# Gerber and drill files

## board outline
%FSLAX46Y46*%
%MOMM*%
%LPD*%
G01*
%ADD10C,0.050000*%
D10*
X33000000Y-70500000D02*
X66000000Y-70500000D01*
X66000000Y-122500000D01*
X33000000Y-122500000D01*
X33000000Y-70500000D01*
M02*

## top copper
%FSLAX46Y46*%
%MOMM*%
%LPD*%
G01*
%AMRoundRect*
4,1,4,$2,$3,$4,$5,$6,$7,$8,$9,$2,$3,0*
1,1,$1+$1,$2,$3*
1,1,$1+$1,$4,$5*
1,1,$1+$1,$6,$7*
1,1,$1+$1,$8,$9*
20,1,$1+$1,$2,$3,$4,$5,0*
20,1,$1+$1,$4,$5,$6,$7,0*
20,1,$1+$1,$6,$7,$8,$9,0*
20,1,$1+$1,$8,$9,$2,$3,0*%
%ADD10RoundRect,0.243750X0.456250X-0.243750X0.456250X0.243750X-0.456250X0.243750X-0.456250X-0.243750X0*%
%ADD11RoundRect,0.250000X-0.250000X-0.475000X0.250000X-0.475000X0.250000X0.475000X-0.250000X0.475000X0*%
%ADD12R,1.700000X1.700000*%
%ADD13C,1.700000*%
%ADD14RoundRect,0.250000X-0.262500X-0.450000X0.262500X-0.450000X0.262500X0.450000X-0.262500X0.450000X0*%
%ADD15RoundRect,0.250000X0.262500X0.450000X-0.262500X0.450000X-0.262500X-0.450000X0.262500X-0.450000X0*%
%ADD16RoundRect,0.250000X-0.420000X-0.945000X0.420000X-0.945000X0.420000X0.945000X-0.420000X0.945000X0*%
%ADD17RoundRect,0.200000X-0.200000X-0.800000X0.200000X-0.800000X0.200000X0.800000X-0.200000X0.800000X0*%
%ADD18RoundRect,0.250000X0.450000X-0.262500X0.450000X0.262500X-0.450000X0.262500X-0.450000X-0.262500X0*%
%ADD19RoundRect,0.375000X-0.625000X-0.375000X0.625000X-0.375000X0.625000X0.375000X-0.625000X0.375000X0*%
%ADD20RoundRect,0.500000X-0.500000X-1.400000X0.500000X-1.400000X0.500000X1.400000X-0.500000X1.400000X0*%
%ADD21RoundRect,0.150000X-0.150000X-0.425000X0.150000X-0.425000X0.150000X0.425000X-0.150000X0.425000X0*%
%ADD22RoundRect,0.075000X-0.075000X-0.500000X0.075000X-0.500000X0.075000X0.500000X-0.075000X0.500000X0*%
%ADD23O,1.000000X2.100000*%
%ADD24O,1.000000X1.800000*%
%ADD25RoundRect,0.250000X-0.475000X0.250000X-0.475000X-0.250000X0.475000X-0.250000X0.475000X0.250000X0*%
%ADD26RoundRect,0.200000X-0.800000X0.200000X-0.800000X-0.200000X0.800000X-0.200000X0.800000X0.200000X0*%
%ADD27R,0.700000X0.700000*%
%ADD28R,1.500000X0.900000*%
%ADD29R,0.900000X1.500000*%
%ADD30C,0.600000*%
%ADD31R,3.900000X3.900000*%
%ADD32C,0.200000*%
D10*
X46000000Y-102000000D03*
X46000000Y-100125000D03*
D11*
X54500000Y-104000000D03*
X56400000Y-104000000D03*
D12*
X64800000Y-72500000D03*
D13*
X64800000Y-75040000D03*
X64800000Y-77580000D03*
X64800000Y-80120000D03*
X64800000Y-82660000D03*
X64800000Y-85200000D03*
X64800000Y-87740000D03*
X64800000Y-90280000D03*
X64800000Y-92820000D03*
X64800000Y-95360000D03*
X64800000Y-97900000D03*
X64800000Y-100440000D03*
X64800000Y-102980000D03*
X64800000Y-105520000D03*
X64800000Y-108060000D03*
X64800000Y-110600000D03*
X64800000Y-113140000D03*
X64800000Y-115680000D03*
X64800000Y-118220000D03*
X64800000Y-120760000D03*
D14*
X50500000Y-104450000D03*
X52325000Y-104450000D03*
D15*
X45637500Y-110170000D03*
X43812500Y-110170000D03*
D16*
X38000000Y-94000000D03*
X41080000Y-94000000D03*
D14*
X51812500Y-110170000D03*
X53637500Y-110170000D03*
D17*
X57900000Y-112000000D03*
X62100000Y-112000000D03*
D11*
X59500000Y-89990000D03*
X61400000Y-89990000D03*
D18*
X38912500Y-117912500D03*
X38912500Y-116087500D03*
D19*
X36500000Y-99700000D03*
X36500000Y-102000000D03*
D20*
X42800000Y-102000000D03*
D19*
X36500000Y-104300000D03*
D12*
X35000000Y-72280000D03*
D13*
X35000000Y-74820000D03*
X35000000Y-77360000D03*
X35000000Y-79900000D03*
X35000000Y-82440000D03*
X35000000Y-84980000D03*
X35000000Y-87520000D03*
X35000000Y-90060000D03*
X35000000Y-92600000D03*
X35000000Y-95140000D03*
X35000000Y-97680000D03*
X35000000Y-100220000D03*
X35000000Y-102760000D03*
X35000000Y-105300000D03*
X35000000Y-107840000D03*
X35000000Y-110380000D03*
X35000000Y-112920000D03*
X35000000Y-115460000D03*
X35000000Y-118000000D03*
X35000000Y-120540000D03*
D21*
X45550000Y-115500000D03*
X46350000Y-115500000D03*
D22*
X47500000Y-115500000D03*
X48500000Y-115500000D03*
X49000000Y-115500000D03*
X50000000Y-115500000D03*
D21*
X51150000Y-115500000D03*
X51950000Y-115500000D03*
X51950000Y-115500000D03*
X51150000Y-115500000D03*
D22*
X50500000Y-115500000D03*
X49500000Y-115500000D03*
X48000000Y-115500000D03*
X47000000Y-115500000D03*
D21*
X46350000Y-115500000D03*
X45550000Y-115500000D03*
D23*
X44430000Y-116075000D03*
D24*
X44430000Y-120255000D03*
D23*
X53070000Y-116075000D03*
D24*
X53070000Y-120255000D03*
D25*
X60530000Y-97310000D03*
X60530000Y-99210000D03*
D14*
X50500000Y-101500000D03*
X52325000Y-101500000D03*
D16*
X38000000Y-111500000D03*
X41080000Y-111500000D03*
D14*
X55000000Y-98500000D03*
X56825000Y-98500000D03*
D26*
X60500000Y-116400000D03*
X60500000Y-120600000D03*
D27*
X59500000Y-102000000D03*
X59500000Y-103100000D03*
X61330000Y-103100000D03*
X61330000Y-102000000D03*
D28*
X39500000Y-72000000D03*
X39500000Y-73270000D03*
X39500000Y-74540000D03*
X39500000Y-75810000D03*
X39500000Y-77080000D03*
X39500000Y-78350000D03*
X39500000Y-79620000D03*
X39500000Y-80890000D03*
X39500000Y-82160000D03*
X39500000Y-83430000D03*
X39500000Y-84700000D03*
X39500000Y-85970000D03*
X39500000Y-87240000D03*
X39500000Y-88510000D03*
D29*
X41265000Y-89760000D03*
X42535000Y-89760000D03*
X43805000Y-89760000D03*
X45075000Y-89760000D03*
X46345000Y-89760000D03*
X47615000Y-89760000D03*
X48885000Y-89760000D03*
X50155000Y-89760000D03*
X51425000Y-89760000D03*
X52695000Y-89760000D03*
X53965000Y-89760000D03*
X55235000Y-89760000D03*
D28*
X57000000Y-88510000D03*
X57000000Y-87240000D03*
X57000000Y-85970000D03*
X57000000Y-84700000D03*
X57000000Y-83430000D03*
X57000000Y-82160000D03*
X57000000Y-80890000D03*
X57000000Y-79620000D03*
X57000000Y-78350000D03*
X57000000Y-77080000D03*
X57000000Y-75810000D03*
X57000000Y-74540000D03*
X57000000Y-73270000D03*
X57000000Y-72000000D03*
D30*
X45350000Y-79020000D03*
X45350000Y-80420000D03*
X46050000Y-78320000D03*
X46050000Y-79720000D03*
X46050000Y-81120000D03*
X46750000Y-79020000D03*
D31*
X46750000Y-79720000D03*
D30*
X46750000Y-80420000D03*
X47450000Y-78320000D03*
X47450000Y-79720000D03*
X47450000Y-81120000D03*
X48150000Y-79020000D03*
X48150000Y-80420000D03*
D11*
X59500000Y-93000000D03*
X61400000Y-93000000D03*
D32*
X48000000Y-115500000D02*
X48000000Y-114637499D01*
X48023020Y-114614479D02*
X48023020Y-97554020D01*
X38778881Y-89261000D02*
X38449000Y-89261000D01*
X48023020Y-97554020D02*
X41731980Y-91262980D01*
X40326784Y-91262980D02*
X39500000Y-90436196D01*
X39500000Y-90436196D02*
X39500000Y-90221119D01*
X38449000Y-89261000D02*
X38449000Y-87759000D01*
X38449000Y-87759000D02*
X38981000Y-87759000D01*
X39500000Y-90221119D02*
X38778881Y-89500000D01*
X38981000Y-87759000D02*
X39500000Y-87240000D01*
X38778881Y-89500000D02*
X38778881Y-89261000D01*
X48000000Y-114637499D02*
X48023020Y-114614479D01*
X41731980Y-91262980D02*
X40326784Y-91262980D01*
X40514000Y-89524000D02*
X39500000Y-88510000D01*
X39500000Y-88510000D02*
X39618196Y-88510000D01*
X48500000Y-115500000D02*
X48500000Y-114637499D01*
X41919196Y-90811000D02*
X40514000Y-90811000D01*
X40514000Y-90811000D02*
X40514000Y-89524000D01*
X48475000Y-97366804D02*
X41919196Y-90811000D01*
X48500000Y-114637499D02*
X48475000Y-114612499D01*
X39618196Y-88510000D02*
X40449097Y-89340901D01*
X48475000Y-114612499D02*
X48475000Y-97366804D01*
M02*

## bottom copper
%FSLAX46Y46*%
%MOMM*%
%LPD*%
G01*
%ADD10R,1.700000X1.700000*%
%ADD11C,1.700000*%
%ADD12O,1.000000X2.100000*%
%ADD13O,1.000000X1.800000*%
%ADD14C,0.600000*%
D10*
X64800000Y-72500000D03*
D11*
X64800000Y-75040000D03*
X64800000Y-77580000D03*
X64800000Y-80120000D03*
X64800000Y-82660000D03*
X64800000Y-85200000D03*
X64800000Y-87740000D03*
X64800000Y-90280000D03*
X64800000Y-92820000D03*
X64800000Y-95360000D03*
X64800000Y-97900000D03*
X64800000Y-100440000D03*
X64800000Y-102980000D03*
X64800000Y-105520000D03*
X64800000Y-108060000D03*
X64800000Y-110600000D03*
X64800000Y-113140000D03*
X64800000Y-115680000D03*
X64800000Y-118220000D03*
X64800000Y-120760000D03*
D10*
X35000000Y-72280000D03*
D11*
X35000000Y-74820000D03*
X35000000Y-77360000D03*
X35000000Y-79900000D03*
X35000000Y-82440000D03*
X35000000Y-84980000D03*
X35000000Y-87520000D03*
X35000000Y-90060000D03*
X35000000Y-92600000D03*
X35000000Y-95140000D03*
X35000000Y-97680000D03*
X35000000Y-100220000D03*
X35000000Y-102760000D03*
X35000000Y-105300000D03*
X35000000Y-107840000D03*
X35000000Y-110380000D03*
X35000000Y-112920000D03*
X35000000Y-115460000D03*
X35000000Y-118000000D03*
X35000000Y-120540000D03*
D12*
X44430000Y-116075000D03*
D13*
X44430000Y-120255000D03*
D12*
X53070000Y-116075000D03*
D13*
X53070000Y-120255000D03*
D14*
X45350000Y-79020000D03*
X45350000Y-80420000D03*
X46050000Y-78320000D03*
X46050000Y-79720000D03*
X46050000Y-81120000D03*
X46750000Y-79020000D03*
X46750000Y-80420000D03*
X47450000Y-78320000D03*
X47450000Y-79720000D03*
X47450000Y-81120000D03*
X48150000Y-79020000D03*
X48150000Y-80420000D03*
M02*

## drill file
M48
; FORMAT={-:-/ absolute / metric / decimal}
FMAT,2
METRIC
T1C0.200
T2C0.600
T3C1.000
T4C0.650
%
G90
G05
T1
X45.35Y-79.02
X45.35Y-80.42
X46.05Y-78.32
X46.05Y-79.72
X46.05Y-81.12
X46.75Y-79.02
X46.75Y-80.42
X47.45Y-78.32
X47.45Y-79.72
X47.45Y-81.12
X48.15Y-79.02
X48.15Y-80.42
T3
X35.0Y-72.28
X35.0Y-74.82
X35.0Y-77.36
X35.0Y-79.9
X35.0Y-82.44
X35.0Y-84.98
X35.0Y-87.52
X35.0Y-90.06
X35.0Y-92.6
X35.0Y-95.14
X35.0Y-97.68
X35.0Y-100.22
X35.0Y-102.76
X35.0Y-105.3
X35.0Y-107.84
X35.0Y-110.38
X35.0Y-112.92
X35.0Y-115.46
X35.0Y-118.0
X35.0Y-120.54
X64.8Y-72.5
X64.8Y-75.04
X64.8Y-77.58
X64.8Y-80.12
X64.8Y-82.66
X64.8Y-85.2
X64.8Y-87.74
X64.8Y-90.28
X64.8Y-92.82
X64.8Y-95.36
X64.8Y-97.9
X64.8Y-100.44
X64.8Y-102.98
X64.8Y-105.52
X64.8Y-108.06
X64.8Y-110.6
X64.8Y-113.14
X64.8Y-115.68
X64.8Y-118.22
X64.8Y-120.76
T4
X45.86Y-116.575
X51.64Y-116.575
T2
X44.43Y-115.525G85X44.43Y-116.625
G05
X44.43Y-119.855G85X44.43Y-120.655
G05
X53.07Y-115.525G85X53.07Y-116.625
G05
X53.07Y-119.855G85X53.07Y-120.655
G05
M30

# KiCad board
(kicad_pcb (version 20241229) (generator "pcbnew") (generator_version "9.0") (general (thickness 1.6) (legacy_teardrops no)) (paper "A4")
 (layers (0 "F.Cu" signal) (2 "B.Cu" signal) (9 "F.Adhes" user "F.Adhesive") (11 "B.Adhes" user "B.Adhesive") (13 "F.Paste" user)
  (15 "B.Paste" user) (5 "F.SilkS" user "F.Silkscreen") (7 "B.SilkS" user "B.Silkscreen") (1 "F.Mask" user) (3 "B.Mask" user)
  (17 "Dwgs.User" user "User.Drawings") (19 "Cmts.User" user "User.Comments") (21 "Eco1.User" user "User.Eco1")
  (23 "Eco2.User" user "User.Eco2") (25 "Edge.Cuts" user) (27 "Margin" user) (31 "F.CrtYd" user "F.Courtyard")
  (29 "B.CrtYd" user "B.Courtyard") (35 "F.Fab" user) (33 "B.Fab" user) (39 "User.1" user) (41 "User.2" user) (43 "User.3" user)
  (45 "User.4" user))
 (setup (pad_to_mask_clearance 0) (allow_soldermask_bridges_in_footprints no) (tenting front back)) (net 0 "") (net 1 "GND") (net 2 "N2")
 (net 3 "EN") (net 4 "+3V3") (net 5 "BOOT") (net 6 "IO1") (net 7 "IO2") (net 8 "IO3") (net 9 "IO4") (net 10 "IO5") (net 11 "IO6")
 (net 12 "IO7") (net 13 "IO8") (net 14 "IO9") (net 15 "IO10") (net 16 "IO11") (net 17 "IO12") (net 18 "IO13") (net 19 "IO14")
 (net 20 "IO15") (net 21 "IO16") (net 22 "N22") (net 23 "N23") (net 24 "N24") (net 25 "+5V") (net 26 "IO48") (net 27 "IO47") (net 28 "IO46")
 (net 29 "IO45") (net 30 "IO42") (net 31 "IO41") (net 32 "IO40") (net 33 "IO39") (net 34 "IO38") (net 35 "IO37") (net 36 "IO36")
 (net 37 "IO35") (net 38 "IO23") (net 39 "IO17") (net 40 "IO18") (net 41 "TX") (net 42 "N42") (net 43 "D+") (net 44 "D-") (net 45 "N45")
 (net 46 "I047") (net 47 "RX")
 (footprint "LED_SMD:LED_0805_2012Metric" (layer "F.Cu") (at 46 101.0625 90)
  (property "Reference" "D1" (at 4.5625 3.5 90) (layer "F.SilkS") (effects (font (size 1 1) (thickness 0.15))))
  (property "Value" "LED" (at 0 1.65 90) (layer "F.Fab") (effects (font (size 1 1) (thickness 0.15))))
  (pad "1" smd roundrect (at -0.9375 0 90) (size 0.975 1.4) (layers "F.Cu" "F.Mask" "F.Paste") (roundrect_rratio 0.25) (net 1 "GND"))
  (pad "2" smd roundrect (at 0.9375 0 90) (size 0.975 1.4) (layers "F.Cu" "F.Mask" "F.Paste") (roundrect_rratio 0.25) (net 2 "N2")))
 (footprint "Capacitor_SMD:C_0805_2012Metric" (layer "F.Cu") (at 55.45 104)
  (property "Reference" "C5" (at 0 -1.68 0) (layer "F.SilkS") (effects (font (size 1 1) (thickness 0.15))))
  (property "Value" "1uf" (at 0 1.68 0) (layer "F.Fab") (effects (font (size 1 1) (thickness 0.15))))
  (pad "1" smd roundrect (at -0.95 0) (size 1 1.45) (layers "F.Cu" "F.Mask" "F.Paste") (roundrect_rratio 0.25) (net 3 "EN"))
  (pad "2" smd roundrect (at 0.95 0) (size 1 1.45) (layers "F.Cu" "F.Mask" "F.Paste") (roundrect_rratio 0.25) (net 1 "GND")))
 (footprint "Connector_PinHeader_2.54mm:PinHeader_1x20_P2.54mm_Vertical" (layer "F.Cu") (at 64.8 72.5)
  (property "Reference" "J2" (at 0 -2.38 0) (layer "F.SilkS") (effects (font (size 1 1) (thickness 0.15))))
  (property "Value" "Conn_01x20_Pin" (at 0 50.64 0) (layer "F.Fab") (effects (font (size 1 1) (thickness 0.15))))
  (pad "1" thru_hole rect (at 0 0) (size 1.7 1.7) (drill 1) (layers "*.Cu" "*.Mask") (remove_unused_layers no) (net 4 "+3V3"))
  (pad "2" thru_hole circle (at 0 2.54) (size 1.7 1.7) (drill 1) (layers "*.Cu" "*.Mask") (remove_unused_layers no) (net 1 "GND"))
  (pad "3" thru_hole circle (at 0 5.08) (size 1.7 1.7) (drill 1) (layers "*.Cu" "*.Mask") (remove_unused_layers no) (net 3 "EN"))
  (pad "4" thru_hole circle (at 0 7.62) (size 1.7 1.7) (drill 1) (layers "*.Cu" "*.Mask") (remove_unused_layers no) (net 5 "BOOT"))
  (pad "5" thru_hole circle (at 0 10.16) (size 1.7 1.7) (drill 1) (layers "*.Cu" "*.Mask") (remove_unused_layers no) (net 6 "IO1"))
  (pad "6" thru_hole circle (at 0 12.7) (size 1.7 1.7) (drill 1) (layers "*.Cu" "*.Mask") (remove_unused_layers no) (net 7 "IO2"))
  (pad "7" thru_hole circle (at 0 15.24) (size 1.7 1.7) (drill 1) (layers "*.Cu" "*.Mask") (remove_unused_layers no) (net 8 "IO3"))
  (pad "8" thru_hole circle (at 0 17.78) (size 1.7 1.7) (drill 1) (layers "*.Cu" "*.Mask") (remove_unused_layers no) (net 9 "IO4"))
  (pad "9" thru_hole circle (at 0 20.32) (size 1.7 1.7) (drill 1) (layers "*.Cu" "*.Mask") (remove_unused_layers no) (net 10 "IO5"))
  (pad "10" thru_hole circle (at 0 22.86) (size 1.7 1.7) (drill 1) (layers "*.Cu" "*.Mask") (remove_unused_layers no) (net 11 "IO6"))
  (pad "11" thru_hole circle (at 0 25.4) (size 1.7 1.7) (drill 1) (layers "*.Cu" "*.Mask") (remove_unused_layers no) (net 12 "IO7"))
  (pad "12" thru_hole circle (at 0 27.94) (size 1.7 1.7) (drill 1) (layers "*.Cu" "*.Mask") (remove_unused_layers no) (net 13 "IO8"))
  (pad "13" thru_hole circle (at 0 30.48) (size 1.7 1.7) (drill 1) (layers "*.Cu" "*.Mask") (remove_unused_layers no) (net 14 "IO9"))
  (pad "14" thru_hole circle (at 0 33.02) (size 1.7 1.7) (drill 1) (layers "*.Cu" "*.Mask") (remove_unused_layers no) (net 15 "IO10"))
  (pad "15" thru_hole circle (at 0 35.56) (size 1.7 1.7) (drill 1) (layers "*.Cu" "*.Mask") (remove_unused_layers no) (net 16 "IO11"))
  (pad "16" thru_hole circle (at 0 38.1) (size 1.7 1.7) (drill 1) (layers "*.Cu" "*.Mask") (remove_unused_layers no) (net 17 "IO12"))
  (pad "17" thru_hole circle (at 0 40.64) (size 1.7 1.7) (drill 1) (layers "*.Cu" "*.Mask") (remove_unused_layers no) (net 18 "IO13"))
  (pad "18" thru_hole circle (at 0 43.18) (size 1.7 1.7) (drill 1) (layers "*.Cu" "*.Mask") (remove_unused_layers no) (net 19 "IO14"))
  (pad "19" thru_hole circle (at 0 45.72) (size 1.7 1.7) (drill 1) (layers "*.Cu" "*.Mask") (remove_unused_layers no) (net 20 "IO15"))
  (pad "20" thru_hole circle (at 0 48.26) (size 1.7 1.7) (drill 1) (layers "*.Cu" "*.Mask") (remove_unused_layers no) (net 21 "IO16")))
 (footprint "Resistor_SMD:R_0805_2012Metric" (layer "F.Cu") (at 51.4125 104.45)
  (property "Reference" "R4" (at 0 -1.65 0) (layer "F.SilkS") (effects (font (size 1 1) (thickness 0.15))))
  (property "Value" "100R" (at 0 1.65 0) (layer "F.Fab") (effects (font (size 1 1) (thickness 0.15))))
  (pad "1" smd roundrect (at -0.9125 0) (size 1.025 1.4) (layers "F.Cu" "F.Mask" "F.Paste") (roundrect_rratio 0.243902) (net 5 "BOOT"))
  (pad "2" smd roundrect (at 0.9125 0) (size 1.025 1.4) (layers "F.Cu" "F.Mask" "F.Paste") (roundrect_rratio 0.243902) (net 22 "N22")))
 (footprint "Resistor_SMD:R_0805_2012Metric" (layer "F.Cu") (at 44.725 110.17 180)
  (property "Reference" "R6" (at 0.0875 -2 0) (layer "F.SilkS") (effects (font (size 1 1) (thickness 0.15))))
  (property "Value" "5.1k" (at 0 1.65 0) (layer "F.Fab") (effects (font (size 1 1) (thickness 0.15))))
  (pad "1" smd roundrect (at -0.9125 0 180) (size 1.025 1.4) (layers "F.Cu" "F.Mask" "F.Paste") (roundrect_rratio 0.243902) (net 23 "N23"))
  (pad "2" smd roundrect (at 0.9125 0 180) (size 1.025 1.4) (layers "F.Cu" "F.Mask" "F.Paste") (roundrect_rratio 0.243902) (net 1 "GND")))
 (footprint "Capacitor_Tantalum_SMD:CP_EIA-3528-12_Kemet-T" (layer "F.Cu") (at 39.54 94)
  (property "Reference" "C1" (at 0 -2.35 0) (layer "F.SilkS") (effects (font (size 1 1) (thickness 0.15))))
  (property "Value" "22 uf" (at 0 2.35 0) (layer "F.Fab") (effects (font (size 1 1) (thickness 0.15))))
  (pad "1" smd roundrect (at -1.54 0) (size 1.34 2.39) (layers "F.Cu" "F.Mask" "F.Paste") (roundrect_rratio 0.186567) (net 4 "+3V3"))
  (pad "2" smd roundrect (at 1.54 0) (size 1.34 2.39) (layers "F.Cu" "F.Mask" "F.Paste") (roundrect_rratio 0.186567) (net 1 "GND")))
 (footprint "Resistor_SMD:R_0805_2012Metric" (layer "F.Cu") (at 52.725 110.17)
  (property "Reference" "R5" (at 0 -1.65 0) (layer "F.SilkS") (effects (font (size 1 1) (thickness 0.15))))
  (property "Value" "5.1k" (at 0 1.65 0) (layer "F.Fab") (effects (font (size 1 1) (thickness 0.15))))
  (pad "1" smd roundrect (at -0.9125 0) (size 1.025 1.4) (layers "F.Cu" "F.Mask" "F.Paste") (roundrect_rratio 0.243902) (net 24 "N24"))
  (pad "2" smd roundrect (at 0.9125 0) (size 1.025 1.4) (layers "F.Cu" "F.Mask" "F.Paste") (roundrect_rratio 0.243902) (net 1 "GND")))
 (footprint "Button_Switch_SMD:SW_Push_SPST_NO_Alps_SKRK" (layer "F.Cu") (at 60 112)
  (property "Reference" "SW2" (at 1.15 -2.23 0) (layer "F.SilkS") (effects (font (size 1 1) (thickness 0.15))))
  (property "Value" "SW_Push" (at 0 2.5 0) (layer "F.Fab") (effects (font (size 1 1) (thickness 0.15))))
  (pad "1" smd roundrect (at -2.1 0) (size 0.8 2) (layers "F.Cu" "F.Mask" "F.Paste") (roundrect_rratio 0.25) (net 22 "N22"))
  (pad "2" smd roundrect (at 2.1 0) (size 0.8 2) (layers "F.Cu" "F.Mask" "F.Paste") (roundrect_rratio 0.25) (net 1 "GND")))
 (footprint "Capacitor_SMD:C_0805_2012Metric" (layer "F.Cu") (at 60.45 89.99)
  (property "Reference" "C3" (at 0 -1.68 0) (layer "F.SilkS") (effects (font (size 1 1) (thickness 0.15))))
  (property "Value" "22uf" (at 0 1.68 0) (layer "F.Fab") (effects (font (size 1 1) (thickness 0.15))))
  (pad "1" smd roundrect (at -0.95 0) (size 1 1.45) (layers "F.Cu" "F.Mask" "F.Paste") (roundrect_rratio 0.25) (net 4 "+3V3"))
  (pad "2" smd roundrect (at 0.95 0) (size 1 1.45) (layers "F.Cu" "F.Mask" "F.Paste") (roundrect_rratio 0.25) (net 1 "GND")))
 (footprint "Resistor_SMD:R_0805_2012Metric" (layer "F.Cu") (at 38.9125 117 90)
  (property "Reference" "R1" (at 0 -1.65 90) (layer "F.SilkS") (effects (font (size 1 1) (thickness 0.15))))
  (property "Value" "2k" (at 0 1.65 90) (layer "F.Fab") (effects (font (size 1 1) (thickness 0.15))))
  (pad "1" smd roundrect (at -0.9125 0 90) (size 1.025 1.4) (layers "F.Cu" "F.Mask" "F.Paste") (roundrect_rratio 0.243902) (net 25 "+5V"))
  (pad "2" smd roundrect (at 0.9125 0 90) (size 1.025 1.4) (layers "F.Cu" "F.Mask" "F.Paste") (roundrect_rratio 0.243902) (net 2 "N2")))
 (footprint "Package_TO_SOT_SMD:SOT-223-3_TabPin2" (layer "F.Cu") (at 39.65 102)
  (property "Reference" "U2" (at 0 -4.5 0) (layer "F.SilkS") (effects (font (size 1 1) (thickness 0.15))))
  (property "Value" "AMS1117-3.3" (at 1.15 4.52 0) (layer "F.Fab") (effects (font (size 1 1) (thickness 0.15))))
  (pad "1" smd roundrect (at -3.15 -2.3) (size 2 1.5) (layers "F.Cu" "F.Mask" "F.Paste") (roundrect_rratio 0.25) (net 1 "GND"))
  (pad "2" smd roundrect (at -3.15 0) (size 2 1.5) (layers "F.Cu" "F.Mask" "F.Paste") (roundrect_rratio 0.25) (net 4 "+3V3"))
  (pad "2" smd roundrect (at 3.15 0) (size 2 3.8) (layers "F.Cu" "F.Mask" "F.Paste") (roundrect_rratio 0.25) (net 4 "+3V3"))
  (pad "3" smd roundrect (at -3.15 2.3) (size 2 1.5) (layers "F.Cu" "F.Mask" "F.Paste") (roundrect_rratio 0.25) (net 25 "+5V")))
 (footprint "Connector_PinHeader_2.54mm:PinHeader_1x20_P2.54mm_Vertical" (layer "F.Cu") (at 35 72.28)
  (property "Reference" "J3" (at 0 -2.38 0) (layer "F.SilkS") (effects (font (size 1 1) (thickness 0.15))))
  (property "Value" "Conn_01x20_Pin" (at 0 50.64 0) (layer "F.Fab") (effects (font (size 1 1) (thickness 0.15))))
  (pad "1" thru_hole rect (at 0 0) (size 1.7 1.7) (drill 1) (layers "*.Cu" "*.Mask") (remove_unused_layers no) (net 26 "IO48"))
  (pad "2" thru_hole circle (at 0 2.54) (size 1.7 1.7) (drill 1) (layers "*.Cu" "*.Mask") (remove_unused_layers no) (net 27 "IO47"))
  (pad "3" thru_hole circle (at 0 5.08) (size 1.7 1.7) (drill 1) (layers "*.Cu" "*.Mask") (remove_unused_layers no) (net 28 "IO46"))
  (pad "4" thru_hole circle (at 0 7.62) (size 1.7 1.7) (drill 1) (layers "*.Cu" "*.Mask") (remove_unused_layers no) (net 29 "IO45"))
  (pad "5" thru_hole circle (at 0 10.16) (size 1.7 1.7) (drill 1) (layers "*.Cu" "*.Mask") (remove_unused_layers no) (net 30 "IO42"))
  (pad "6" thru_hole circle (at 0 12.7) (size 1.7 1.7) (drill 1) (layers "*.Cu" "*.Mask") (remove_unused_layers no) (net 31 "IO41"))
  (pad "7" thru_hole circle (at 0 15.24) (size 1.7 1.7) (drill 1) (layers "*.Cu" "*.Mask") (remove_unused_layers no) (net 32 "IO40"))
  (pad "8" thru_hole circle (at 0 17.78) (size 1.7 1.7) (drill 1) (layers "*.Cu" "*.Mask") (remove_unused_layers no) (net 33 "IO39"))
  (pad "9" thru_hole circle (at 0 20.32) (size 1.7 1.7) (drill 1) (layers "*.Cu" "*.Mask") (remove_unused_layers no) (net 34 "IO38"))
  (pad "10" thru_hole circle (at 0 22.86) (size 1.7 1.7) (drill 1) (layers "*.Cu" "*.Mask") (remove_unused_layers no) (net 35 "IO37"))
  (pad "11" thru_hole circle (at 0 25.4) (size 1.7 1.7) (drill 1) (layers "*.Cu" "*.Mask") (remove_unused_layers no) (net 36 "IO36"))
  (pad "12" thru_hole circle (at 0 27.94) (size 1.7 1.7) (drill 1) (layers "*.Cu" "*.Mask") (remove_unused_layers no) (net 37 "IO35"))
  (pad "13" thru_hole circle (at 0 30.48) (size 1.7 1.7) (drill 1) (layers "*.Cu" "*.Mask") (remove_unused_layers no) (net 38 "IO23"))
  (pad "14" thru_hole circle (at 0 33.02) (size 1.7 1.7) (drill 1) (layers "*.Cu" "*.Mask") (remove_unused_layers no) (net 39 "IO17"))
  (pad "15" thru_hole circle (at 0 35.56) (size 1.7 1.7) (drill 1) (layers "*.Cu" "*.Mask") (remove_unused_layers no) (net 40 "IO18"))
  (pad "16" thru_hole circle (at 0 38.1) (size 1.7 1.7) (drill 1) (layers "*.Cu" "*.Mask") (remove_unused_layers no) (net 1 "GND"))
  (pad "17" thru_hole circle (at 0 40.64) (size 1.7 1.7) (drill 1) (layers "*.Cu" "*.Mask") (remove_unused_layers no) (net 1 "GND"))
  (pad "18" thru_hole circle (at 0 43.18) (size 1.7 1.7) (drill 1) (layers "*.Cu" "*.Mask") (remove_unused_layers no) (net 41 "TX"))
  (pad "19" thru_hole circle (at 0 45.72) (size 1.7 1.7) (drill 1) (layers "*.Cu" "*.Mask") (remove_unused_layers no) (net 1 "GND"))
  (pad "20" thru_hole circle (at 0 48.26) (size 1.7 1.7) (drill 1) (layers "*.Cu" "*.Mask") (remove_unused_layers no) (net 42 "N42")))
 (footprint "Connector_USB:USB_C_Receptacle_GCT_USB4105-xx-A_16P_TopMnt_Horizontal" (layer "F.Cu") (at 48.75 119.18)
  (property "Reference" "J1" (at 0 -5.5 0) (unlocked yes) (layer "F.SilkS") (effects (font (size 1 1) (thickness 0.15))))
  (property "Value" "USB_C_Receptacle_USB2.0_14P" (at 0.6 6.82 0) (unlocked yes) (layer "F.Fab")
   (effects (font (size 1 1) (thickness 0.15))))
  (pad "" np_thru_hole circle (at -2.89 -2.605) (size 0.65 0.65) (drill 0.65) (layers "*.Cu" "*.Mask"))
  (pad "" np_thru_hole circle (at 2.89 -2.605) (size 0.65 0.65) (drill 0.65) (layers "*.Cu" "*.Mask"))
  (pad "A1" smd roundrect (at -3.2 -3.68) (size 0.6 1.15) (layers "F.Cu" "F.Mask" "F.Paste") (roundrect_rratio 0.25) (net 1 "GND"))
  (pad "A4" smd roundrect (at -2.4 -3.68) (size 0.6 1.15) (layers "F.Cu" "F.Mask" "F.Paste") (roundrect_rratio 0.25) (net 25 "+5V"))
  (pad "A5" smd roundrect (at -1.25 -3.68) (size 0.3 1.15) (layers "F.Cu" "F.Mask" "F.Paste") (roundrect_rratio 0.25) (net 23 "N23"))
  (pad "A6" smd roundrect (at -0.25 -3.68) (size 0.3 1.15) (layers "F.Cu" "F.Mask" "F.Paste") (roundrect_rratio 0.25) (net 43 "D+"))
  (pad "A7" smd roundrect (at 0.25 -3.68) (size 0.3 1.15) (layers "F.Cu" "F.Mask" "F.Paste") (roundrect_rratio 0.25) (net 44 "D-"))
  (pad "A8" smd roundrect (at 1.25 -3.68) (size 0.3 1.15) (layers "F.Cu" "F.Mask" "F.Paste") (roundrect_rratio 0.25))
  (pad "A9" smd roundrect (at 2.4 -3.68) (size 0.6 1.15) (layers "F.Cu" "F.Mask" "F.Paste") (roundrect_rratio 0.25) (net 25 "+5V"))
  (pad "A12" smd roundrect (at 3.2 -3.68) (size 0.6 1.15) (layers "F.Cu" "F.Mask" "F.Paste") (roundrect_rratio 0.25) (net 1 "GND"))
  (pad "B1" smd roundrect (at 3.2 -3.68) (size 0.6 1.15) (layers "F.Cu" "F.Mask" "F.Paste") (roundrect_rratio 0.25) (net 1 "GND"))
  (pad "B4" smd roundrect (at 2.4 -3.68) (size 0.6 1.15) (layers "F.Cu" "F.Mask" "F.Paste") (roundrect_rratio 0.25) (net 25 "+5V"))
  (pad "B5" smd roundrect (at 1.75 -3.68) (size 0.3 1.15) (layers "F.Cu" "F.Mask" "F.Paste") (roundrect_rratio 0.25) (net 24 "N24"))
  (pad "B6" smd roundrect (at 0.75 -3.68) (size 0.3 1.15) (layers "F.Cu" "F.Mask" "F.Paste") (roundrect_rratio 0.25) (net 43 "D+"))
  (pad "B7" smd roundrect (at -0.75 -3.68) (size 0.3 1.15) (layers "F.Cu" "F.Mask" "F.Paste") (roundrect_rratio 0.25) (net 44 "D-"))
  (pad "B8" smd roundrect (at -1.75 -3.68) (size 0.3 1.15) (layers "F.Cu" "F.Mask" "F.Paste") (roundrect_rratio 0.25))
  (pad "B9" smd roundrect (at -2.4 -3.68) (size 0.6 1.15) (layers "F.Cu" "F.Mask" "F.Paste") (roundrect_rratio 0.25) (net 25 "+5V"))
  (pad "B12" smd roundrect (at -3.2 -3.68) (size 0.6 1.15) (layers "F.Cu" "F.Mask" "F.Paste") (roundrect_rratio 0.25) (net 1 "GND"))
  (pad "S1" thru_hole oval (at -4.32 -3.105) (size 1 2.1) (drill oval 0.6 1.7) (layers "*.Cu" "*.Mask" "F.Paste") (remove_unused_layers no)
   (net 1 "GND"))
  (pad "S1" thru_hole oval (at -4.32 1.075) (size 1 1.8) (drill oval 0.6 1.4) (layers "*.Cu" "*.Mask" "F.Paste") (remove_unused_layers no)
   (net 1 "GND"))
  (pad "S1" thru_hole oval (at 4.32 -3.105) (size 1 2.1) (drill oval 0.6 1.7) (layers "*.Cu" "*.Mask" "F.Paste") (remove_unused_layers no)
   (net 1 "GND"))
  (pad "S1" thru_hole oval (at 4.32 1.075) (size 1 1.8) (drill oval 0.6 1.4) (layers "*.Cu" "*.Mask" "F.Paste") (remove_unused_layers no)
   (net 1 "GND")))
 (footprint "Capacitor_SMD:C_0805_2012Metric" (layer "F.Cu") (at 60.53 98.26 -90)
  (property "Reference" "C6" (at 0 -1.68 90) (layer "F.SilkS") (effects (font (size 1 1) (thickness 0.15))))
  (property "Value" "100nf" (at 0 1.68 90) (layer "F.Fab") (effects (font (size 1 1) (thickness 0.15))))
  (pad "1" smd roundrect (at -0.95 0 270) (size 1 1.45) (layers "F.Cu" "F.Mask" "F.Paste") (roundrect_rratio 0.25) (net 3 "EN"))
  (pad "2" smd roundrect (at 0.95 0 270) (size 1 1.45) (layers "F.Cu" "F.Mask" "F.Paste") (roundrect_rratio 0.25) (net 1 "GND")))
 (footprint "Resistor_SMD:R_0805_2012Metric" (layer "F.Cu") (at 51.4125 101.5)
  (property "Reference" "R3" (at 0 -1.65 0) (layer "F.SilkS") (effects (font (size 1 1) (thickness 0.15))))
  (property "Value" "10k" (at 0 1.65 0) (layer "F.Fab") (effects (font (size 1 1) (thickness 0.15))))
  (pad "1" smd roundrect (at -0.9125 0) (size 1.025 1.4) (layers "F.Cu" "F.Mask" "F.Paste") (roundrect_rratio 0.243902) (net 4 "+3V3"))
  (pad "2" smd roundrect (at 0.9125 0) (size 1.025 1.4) (layers "F.Cu" "F.Mask" "F.Paste") (roundrect_rratio 0.243902) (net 5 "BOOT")))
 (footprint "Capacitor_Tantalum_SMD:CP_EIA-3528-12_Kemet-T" (layer "F.Cu") (at 39.54 111.5)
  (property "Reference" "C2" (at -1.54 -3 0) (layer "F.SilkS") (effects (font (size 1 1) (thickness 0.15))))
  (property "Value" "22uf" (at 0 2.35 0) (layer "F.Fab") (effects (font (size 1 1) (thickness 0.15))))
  (pad "1" smd roundrect (at -1.54 0) (size 1.34 2.39) (layers "F.Cu" "F.Mask" "F.Paste") (roundrect_rratio 0.186567) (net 25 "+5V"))
  (pad "2" smd roundrect (at 1.54 0) (size 1.34 2.39) (layers "F.Cu" "F.Mask" "F.Paste") (roundrect_rratio 0.186567) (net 1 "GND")))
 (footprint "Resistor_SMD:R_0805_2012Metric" (layer "F.Cu") (at 55.9125 98.5)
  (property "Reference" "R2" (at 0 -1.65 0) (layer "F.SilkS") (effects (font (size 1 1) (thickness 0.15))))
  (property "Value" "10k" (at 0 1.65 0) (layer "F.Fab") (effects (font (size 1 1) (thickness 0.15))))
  (pad "1" smd roundrect (at -0.9125 0) (size 1.025 1.4) (layers "F.Cu" "F.Mask" "F.Paste") (roundrect_rratio 0.243902) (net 4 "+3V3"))
  (pad "2" smd roundrect (at 0.9125 0) (size 1.025 1.4) (layers "F.Cu" "F.Mask" "F.Paste") (roundrect_rratio 0.243902) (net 3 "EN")))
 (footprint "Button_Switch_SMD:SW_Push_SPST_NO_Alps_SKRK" (layer "F.Cu") (at 60.5 118.5 -90)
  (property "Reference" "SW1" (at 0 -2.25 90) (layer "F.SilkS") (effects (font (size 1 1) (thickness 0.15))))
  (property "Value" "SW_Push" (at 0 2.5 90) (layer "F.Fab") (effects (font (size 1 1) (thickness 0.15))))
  (pad "1" smd roundrect (at -2.1 0 270) (size 0.8 2) (layers "F.Cu" "F.Mask" "F.Paste") (roundrect_rratio 0.25) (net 3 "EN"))
  (pad "2" smd roundrect (at 2.1 0 270) (size 0.8 2) (layers "F.Cu" "F.Mask" "F.Paste") (roundrect_rratio 0.25) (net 1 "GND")))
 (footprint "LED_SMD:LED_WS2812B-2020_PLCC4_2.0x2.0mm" (layer "F.Cu") (at 60.415 102.55)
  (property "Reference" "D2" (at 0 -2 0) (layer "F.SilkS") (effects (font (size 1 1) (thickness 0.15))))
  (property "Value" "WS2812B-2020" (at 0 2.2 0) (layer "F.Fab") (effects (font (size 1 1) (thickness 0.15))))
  (pad "1" smd rect (at -0.915 -0.55) (size 0.7 0.7) (layers "F.Cu" "F.Mask" "F.Paste") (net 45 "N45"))
  (pad "2" smd rect (at -0.915 0.55) (size 0.7 0.7) (layers "F.Cu" "F.Mask" "F.Paste") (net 1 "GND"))
  (pad "3" smd rect (at 0.915 0.55) (size 0.7 0.7) (layers "F.Cu" "F.Mask" "F.Paste") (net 26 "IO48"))
  (pad "4" smd rect (at 0.915 -0.55) (size 0.7 0.7) (layers "F.Cu" "F.Mask" "F.Paste") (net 4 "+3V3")))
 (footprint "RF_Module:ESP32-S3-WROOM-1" (layer "F.Cu") (at 48.25 77.26)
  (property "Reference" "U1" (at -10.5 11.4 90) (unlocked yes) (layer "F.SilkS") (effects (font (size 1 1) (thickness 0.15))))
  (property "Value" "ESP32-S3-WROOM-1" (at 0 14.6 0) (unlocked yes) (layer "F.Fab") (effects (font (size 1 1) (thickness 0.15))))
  (pad "" smd rect (at -2.9 1.06) (size 0.9 0.9) (layers "F.Paste"))
  (pad "" smd rect (at -2.9 2.46 270) (size 0.9 0.9) (layers "F.Paste"))
  (pad "" smd rect (at -2.9 3.86) (size 0.9 0.9) (layers "F.Paste"))
  (pad "" smd rect (at -1.5 1.06 270) (size 0.9 0.9) (layers "F.Paste"))
  (pad "" smd rect (at -1.5 2.46 270) (size 0.9 0.9) (layers "F.Paste"))
  (pad "" smd rect (at -1.5 3.86 270) (size 0.9 0.9) (layers "F.Paste"))
  (pad "" smd rect (at -0.1 1.06 270) (size 0.9 0.9) (layers "F.Paste"))
  (pad "" smd rect (at -0.1 2.46 270) (size 0.9 0.9) (layers "F.Paste"))
  (pad "" smd rect (at -0.1 3.86 270) (size 0.9 0.9) (layers "F.Paste"))
  (pad "1" smd rect (at -8.75 -5.26) (size 1.5 0.9) (layers "F.Cu" "F.Mask" "F.Paste") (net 1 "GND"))
  (pad "2" smd rect (at -8.75 -3.99) (size 1.5 0.9) (layers "F.Cu" "F.Mask" "F.Paste") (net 4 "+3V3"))
  (pad "3" smd rect (at -8.75 -2.72) (size 1.5 0.9) (layers "F.Cu" "F.Mask" "F.Paste") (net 3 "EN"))
  (pad "4" smd rect (at -8.75 -1.45) (size 1.5 0.9) (layers "F.Cu" "F.Mask" "F.Paste") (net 9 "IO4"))
  (pad "5" smd rect (at -8.75 -0.18) (size 1.5 0.9) (layers "F.Cu" "F.Mask" "F.Paste") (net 10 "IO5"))
  (pad "6" smd rect (at -8.75 1.09) (size 1.5 0.9) (layers "F.Cu" "F.Mask" "F.Paste") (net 11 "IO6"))
  (pad "7" smd rect (at -8.75 2.36) (size 1.5 0.9) (layers "F.Cu" "F.Mask" "F.Paste") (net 12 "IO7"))
  (pad "8" smd rect (at -8.75 3.63) (size 1.5 0.9) (layers "F.Cu" "F.Mask" "F.Paste") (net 20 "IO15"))
  (pad "9" smd rect (at -8.75 4.9) (size 1.5 0.9) (layers "F.Cu" "F.Mask" "F.Paste") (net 21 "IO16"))
  (pad "10" smd rect (at -8.75 6.17) (size 1.5 0.9) (layers "F.Cu" "F.Mask" "F.Paste") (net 39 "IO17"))
  (pad "11" smd rect (at -8.75 7.44) (size 1.5 0.9) (layers "F.Cu" "F.Mask" "F.Paste") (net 40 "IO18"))
  (pad "12" smd rect (at -8.75 8.71) (size 1.5 0.9) (layers "F.Cu" "F.Mask" "F.Paste") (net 13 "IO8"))
  (pad "13" smd rect (at -8.75 9.98) (size 1.5 0.9) (layers "F.Cu" "F.Mask" "F.Paste") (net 44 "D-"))
  (pad "14" smd rect (at -8.75 11.25 180) (size 1.5 0.9) (layers "F.Cu" "F.Mask" "F.Paste") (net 43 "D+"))
  (pad "15" smd rect (at -6.985 12.5 270) (size 1.5 0.9) (layers "F.Cu" "F.Mask" "F.Paste") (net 8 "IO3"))
  (pad "16" smd rect (at -5.715 12.5 270) (size 1.5 0.9) (layers "F.Cu" "F.Mask" "F.Paste") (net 28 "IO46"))
  (pad "17" smd rect (at -4.445 12.5 270) (size 1.5 0.9) (layers "F.Cu" "F.Mask" "F.Paste") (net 14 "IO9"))
  (pad "18" smd rect (at -3.175 12.5 270) (size 1.5 0.9) (layers "F.Cu" "F.Mask" "F.Paste") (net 15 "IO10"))
  (pad "19" smd rect (at -1.905 12.5 270) (size 1.5 0.9) (layers "F.Cu" "F.Mask" "F.Paste") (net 16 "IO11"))
  (pad "20" smd rect (at -0.635 12.5 270) (size 1.5 0.9) (layers "F.Cu" "F.Mask" "F.Paste") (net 17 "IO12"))
  (pad "21" smd rect (at 0.635 12.5 270) (size 1.5 0.9) (layers "F.Cu" "F.Mask" "F.Paste") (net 18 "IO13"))
  (pad "22" smd rect (at 1.905 12.5 270) (size 1.5 0.9) (layers "F.Cu" "F.Mask" "F.Paste") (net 19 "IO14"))
  (pad "23" smd rect (at 3.175 12.5 270) (size 1.5 0.9) (layers "F.Cu" "F.Mask" "F.Paste") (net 38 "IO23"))
  (pad "24" smd rect (at 4.445 12.5 270) (size 1.5 0.9) (layers "F.Cu" "F.Mask" "F.Paste") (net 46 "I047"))
  (pad "25" smd rect (at 5.715 12.5 270) (size 1.5 0.9) (layers "F.Cu" "F.Mask" "F.Paste") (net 26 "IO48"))
  (pad "26" smd rect (at 6.985 12.5 270) (size 1.5 0.9) (layers "F.Cu" "F.Mask" "F.Paste") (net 29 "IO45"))
  (pad "27" smd rect (at 8.75 11.25) (size 1.5 0.9) (layers "F.Cu" "F.Mask" "F.Paste") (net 5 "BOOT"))
  (pad "28" smd rect (at 8.75 9.98) (size 1.5 0.9) (layers "F.Cu" "F.Mask" "F.Paste") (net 37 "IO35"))
  (pad "29" smd rect (at 8.75 8.71) (size 1.5 0.9) (layers "F.Cu" "F.Mask" "F.Paste") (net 36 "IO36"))
  (pad "30" smd rect (at 8.75 7.44) (size 1.5 0.9) (layers "F.Cu" "F.Mask" "F.Paste") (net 35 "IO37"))
  (pad "31" smd rect (at 8.75 6.17) (size 1.5 0.9) (layers "F.Cu" "F.Mask" "F.Paste") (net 34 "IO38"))
  (pad "32" smd rect (at 8.75 4.9) (size 1.5 0.9) (layers "F.Cu" "F.Mask" "F.Paste") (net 33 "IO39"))
  (pad "33" smd rect (at 8.75 3.63) (size 1.5 0.9) (layers "F.Cu" "F.Mask" "F.Paste") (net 32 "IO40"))
  (pad "34" smd rect (at 8.75 2.36) (size 1.5 0.9) (layers "F.Cu" "F.Mask" "F.Paste") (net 31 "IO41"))
  (pad "35" smd rect (at 8.75 1.09) (size 1.5 0.9) (layers "F.Cu" "F.Mask" "F.Paste") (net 30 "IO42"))
  (pad "36" smd rect (at 8.75 -0.18) (size 1.5 0.9) (layers "F.Cu" "F.Mask" "F.Paste") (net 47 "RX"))
  (pad "37" smd rect (at 8.75 -1.45) (size 1.5 0.9) (layers "F.Cu" "F.Mask" "F.Paste") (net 41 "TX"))
  (pad "38" smd rect (at 8.75 -2.72) (size 1.5 0.9) (layers "F.Cu" "F.Mask" "F.Paste") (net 7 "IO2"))
  (pad "39" smd rect (at 8.75 -3.99) (size 1.5 0.9) (layers "F.Cu" "F.Mask" "F.Paste") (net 6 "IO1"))
  (pad "40" smd rect (at 8.75 -5.26) (size 1.5 0.9) (layers "F.Cu" "F.Mask" "F.Paste") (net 1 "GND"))
  (pad "41" thru_hole circle (at -2.9 1.76 90) (size 0.6 0.6) (drill 0.2) (layers "*.Cu" "F.Mask") (remove_unused_layers no) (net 1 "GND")
   (zone_connect 2))
  (pad "41" thru_hole circle (at -2.9 3.16) (size 0.6 0.6) (drill 0.2) (layers "*.Cu" "F.Mask") (remove_unused_layers no) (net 1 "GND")
   (zone_connect 2))
  (pad "41" thru_hole circle (at -2.2 1.06) (size 0.6 0.6) (drill 0.2) (layers "*.Cu" "F.Mask") (remove_unused_layers no) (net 1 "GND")
   (zone_connect 2))
  (pad "41" thru_hole circle (at -2.2 2.46) (size 0.6 0.6) (drill 0.2) (layers "*.Cu" "F.Mask") (remove_unused_layers no) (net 1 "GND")
   (zone_connect 2))
  (pad "41" thru_hole circle (at -2.2 3.86) (size 0.6 0.6) (drill 0.2) (layers "*.Cu" "F.Mask") (remove_unused_layers no) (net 1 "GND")
   (zone_connect 2))
  (pad "41" thru_hole circle (at -1.5 1.76) (size 0.6 0.6) (drill 0.2) (layers "*.Cu" "F.Mask") (remove_unused_layers no) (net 1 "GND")
   (zone_connect 2))
  (pad "41" smd rect (at -1.5 2.46 270) (size 3.9 3.9) (layers "F.Cu" "F.Mask") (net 1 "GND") (zone_connect 2))
  (pad "41" thru_hole circle (at -1.5 3.16) (size 0.6 0.6) (drill 0.2) (layers "*.Cu" "F.Mask") (remove_unused_layers no) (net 1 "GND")
   (zone_connect 2))
  (pad "41" thru_hole circle (at -0.8 1.06) (size 0.6 0.6) (drill 0.2) (layers "*.Cu" "F.Mask") (remove_unused_layers no) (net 1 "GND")
   (zone_connect 2))
  (pad "41" thru_hole circle (at -0.8 2.46) (size 0.6 0.6) (drill 0.2) (layers "*.Cu" "F.Mask") (remove_unused_layers no) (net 1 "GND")
   (zone_connect 2))
  (pad "41" thru_hole circle (at -0.8 3.86) (size 0.6 0.6) (drill 0.2) (layers "*.Cu" "F.Mask") (remove_unused_layers no) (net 1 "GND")
   (zone_connect 2))
  (pad "41" thru_hole circle (at -0.1 1.76) (size 0.6 0.6) (drill 0.2) (layers "*.Cu" "F.Mask") (remove_unused_layers no) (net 1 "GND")
   (zone_connect 2))
  (pad "41" thru_hole circle (at -0.1 3.16) (size 0.6 0.6) (drill 0.2) (layers "*.Cu" "F.Mask") (remove_unused_layers no) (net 1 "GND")
   (zone_connect 2))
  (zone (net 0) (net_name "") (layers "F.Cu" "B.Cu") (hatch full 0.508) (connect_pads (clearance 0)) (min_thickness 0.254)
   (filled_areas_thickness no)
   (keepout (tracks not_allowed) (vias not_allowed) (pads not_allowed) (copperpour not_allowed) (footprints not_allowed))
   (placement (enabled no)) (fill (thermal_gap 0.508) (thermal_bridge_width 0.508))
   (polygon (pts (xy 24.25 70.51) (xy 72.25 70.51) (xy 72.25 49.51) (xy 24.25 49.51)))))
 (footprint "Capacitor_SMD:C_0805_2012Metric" (layer "F.Cu") (at 60.45 93)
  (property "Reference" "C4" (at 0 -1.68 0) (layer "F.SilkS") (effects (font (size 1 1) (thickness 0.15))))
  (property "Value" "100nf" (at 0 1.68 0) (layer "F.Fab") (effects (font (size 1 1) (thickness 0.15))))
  (pad "1" smd roundrect (at -0.95 0) (size 1 1.45) (layers "F.Cu" "F.Mask" "F.Paste") (roundrect_rratio 0.25) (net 4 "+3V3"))
  (pad "2" smd roundrect (at 0.95 0) (size 1 1.45) (layers "F.Cu" "F.Mask" "F.Paste") (roundrect_rratio 0.25) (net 1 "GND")))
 (gr_rect (start 33 70.5) (end 66 122.5) (stroke (width 0.05) (type solid)) (fill no) (layer "Edge.Cuts"))
 (segment (start 48 115.5) (end 48 114.637499) (width 0.2) (layer "F.Cu") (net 44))
 (segment (start 48.02302 114.614479) (end 48.02302 97.55402) (width 0.2) (layer "F.Cu") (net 44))
 (segment (start 38.778881 89.261) (end 38.449 89.261) (width 0.2) (layer "F.Cu") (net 44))
 (segment (start 48.02302 97.55402) (end 41.73198 91.26298) (width 0.2) (layer "F.Cu") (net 44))
 (segment (start 40.326784 91.26298) (end 39.5 90.436196) (width 0.2) (layer "F.Cu") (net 44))
 (segment (start 39.5 90.436196) (end 39.5 90.221119) (width 0.2) (layer "F.Cu") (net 44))
 (segment (start 38.449 89.261) (end 38.449 87.759) (width 0.2) (layer "F.Cu") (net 44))
 (segment (start 38.449 87.759) (end 38.981 87.759) (width 0.2) (layer "F.Cu") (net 44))
 (segment (start 39.5 90.221119) (end 38.778881 89.5) (width 0.2) (layer "F.Cu") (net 44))
 (segment (start 38.981 87.759) (end 39.5 87.24) (width 0.2) (layer "F.Cu") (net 44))
 (segment (start 38.778881 89.5) (end 38.778881 89.261) (width 0.2) (layer "F.Cu") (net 44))
 (segment (start 48 114.637499) (end 48.02302 114.614479) (width 0.2) (layer "F.Cu") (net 44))
 (segment (start 41.73198 91.26298) (end 40.326784 91.26298) (width 0.2) (layer "F.Cu") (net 44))
 (segment (start 40.514 89.524) (end 39.5 88.51) (width 0.2) (layer "F.Cu") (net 43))
 (segment (start 39.5 88.51) (end 39.618196 88.51) (width 0.2) (layer "F.Cu") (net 43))
 (segment (start 48.5 115.5) (end 48.5 114.637499) (width 0.2) (layer "F.Cu") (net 43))
 (segment (start 41.919196 90.811) (end 40.514 90.811) (width 0.2) (layer "F.Cu") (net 43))
 (segment (start 40.514 90.811) (end 40.514 89.524) (width 0.2) (layer "F.Cu") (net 43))
 (segment (start 48.475 97.366804) (end 41.919196 90.811) (width 0.2) (layer "F.Cu") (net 43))
 (segment (start 48.5 114.637499) (end 48.475 114.612499) (width 0.2) (layer "F.Cu") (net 43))
 (segment (start 39.618196 88.51) (end 40.449097 89.340901) (width 0.2) (layer "F.Cu") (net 43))
 (segment (start 48.475 114.612499) (end 48.475 97.366804) (width 0.2) (layer "F.Cu") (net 43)))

